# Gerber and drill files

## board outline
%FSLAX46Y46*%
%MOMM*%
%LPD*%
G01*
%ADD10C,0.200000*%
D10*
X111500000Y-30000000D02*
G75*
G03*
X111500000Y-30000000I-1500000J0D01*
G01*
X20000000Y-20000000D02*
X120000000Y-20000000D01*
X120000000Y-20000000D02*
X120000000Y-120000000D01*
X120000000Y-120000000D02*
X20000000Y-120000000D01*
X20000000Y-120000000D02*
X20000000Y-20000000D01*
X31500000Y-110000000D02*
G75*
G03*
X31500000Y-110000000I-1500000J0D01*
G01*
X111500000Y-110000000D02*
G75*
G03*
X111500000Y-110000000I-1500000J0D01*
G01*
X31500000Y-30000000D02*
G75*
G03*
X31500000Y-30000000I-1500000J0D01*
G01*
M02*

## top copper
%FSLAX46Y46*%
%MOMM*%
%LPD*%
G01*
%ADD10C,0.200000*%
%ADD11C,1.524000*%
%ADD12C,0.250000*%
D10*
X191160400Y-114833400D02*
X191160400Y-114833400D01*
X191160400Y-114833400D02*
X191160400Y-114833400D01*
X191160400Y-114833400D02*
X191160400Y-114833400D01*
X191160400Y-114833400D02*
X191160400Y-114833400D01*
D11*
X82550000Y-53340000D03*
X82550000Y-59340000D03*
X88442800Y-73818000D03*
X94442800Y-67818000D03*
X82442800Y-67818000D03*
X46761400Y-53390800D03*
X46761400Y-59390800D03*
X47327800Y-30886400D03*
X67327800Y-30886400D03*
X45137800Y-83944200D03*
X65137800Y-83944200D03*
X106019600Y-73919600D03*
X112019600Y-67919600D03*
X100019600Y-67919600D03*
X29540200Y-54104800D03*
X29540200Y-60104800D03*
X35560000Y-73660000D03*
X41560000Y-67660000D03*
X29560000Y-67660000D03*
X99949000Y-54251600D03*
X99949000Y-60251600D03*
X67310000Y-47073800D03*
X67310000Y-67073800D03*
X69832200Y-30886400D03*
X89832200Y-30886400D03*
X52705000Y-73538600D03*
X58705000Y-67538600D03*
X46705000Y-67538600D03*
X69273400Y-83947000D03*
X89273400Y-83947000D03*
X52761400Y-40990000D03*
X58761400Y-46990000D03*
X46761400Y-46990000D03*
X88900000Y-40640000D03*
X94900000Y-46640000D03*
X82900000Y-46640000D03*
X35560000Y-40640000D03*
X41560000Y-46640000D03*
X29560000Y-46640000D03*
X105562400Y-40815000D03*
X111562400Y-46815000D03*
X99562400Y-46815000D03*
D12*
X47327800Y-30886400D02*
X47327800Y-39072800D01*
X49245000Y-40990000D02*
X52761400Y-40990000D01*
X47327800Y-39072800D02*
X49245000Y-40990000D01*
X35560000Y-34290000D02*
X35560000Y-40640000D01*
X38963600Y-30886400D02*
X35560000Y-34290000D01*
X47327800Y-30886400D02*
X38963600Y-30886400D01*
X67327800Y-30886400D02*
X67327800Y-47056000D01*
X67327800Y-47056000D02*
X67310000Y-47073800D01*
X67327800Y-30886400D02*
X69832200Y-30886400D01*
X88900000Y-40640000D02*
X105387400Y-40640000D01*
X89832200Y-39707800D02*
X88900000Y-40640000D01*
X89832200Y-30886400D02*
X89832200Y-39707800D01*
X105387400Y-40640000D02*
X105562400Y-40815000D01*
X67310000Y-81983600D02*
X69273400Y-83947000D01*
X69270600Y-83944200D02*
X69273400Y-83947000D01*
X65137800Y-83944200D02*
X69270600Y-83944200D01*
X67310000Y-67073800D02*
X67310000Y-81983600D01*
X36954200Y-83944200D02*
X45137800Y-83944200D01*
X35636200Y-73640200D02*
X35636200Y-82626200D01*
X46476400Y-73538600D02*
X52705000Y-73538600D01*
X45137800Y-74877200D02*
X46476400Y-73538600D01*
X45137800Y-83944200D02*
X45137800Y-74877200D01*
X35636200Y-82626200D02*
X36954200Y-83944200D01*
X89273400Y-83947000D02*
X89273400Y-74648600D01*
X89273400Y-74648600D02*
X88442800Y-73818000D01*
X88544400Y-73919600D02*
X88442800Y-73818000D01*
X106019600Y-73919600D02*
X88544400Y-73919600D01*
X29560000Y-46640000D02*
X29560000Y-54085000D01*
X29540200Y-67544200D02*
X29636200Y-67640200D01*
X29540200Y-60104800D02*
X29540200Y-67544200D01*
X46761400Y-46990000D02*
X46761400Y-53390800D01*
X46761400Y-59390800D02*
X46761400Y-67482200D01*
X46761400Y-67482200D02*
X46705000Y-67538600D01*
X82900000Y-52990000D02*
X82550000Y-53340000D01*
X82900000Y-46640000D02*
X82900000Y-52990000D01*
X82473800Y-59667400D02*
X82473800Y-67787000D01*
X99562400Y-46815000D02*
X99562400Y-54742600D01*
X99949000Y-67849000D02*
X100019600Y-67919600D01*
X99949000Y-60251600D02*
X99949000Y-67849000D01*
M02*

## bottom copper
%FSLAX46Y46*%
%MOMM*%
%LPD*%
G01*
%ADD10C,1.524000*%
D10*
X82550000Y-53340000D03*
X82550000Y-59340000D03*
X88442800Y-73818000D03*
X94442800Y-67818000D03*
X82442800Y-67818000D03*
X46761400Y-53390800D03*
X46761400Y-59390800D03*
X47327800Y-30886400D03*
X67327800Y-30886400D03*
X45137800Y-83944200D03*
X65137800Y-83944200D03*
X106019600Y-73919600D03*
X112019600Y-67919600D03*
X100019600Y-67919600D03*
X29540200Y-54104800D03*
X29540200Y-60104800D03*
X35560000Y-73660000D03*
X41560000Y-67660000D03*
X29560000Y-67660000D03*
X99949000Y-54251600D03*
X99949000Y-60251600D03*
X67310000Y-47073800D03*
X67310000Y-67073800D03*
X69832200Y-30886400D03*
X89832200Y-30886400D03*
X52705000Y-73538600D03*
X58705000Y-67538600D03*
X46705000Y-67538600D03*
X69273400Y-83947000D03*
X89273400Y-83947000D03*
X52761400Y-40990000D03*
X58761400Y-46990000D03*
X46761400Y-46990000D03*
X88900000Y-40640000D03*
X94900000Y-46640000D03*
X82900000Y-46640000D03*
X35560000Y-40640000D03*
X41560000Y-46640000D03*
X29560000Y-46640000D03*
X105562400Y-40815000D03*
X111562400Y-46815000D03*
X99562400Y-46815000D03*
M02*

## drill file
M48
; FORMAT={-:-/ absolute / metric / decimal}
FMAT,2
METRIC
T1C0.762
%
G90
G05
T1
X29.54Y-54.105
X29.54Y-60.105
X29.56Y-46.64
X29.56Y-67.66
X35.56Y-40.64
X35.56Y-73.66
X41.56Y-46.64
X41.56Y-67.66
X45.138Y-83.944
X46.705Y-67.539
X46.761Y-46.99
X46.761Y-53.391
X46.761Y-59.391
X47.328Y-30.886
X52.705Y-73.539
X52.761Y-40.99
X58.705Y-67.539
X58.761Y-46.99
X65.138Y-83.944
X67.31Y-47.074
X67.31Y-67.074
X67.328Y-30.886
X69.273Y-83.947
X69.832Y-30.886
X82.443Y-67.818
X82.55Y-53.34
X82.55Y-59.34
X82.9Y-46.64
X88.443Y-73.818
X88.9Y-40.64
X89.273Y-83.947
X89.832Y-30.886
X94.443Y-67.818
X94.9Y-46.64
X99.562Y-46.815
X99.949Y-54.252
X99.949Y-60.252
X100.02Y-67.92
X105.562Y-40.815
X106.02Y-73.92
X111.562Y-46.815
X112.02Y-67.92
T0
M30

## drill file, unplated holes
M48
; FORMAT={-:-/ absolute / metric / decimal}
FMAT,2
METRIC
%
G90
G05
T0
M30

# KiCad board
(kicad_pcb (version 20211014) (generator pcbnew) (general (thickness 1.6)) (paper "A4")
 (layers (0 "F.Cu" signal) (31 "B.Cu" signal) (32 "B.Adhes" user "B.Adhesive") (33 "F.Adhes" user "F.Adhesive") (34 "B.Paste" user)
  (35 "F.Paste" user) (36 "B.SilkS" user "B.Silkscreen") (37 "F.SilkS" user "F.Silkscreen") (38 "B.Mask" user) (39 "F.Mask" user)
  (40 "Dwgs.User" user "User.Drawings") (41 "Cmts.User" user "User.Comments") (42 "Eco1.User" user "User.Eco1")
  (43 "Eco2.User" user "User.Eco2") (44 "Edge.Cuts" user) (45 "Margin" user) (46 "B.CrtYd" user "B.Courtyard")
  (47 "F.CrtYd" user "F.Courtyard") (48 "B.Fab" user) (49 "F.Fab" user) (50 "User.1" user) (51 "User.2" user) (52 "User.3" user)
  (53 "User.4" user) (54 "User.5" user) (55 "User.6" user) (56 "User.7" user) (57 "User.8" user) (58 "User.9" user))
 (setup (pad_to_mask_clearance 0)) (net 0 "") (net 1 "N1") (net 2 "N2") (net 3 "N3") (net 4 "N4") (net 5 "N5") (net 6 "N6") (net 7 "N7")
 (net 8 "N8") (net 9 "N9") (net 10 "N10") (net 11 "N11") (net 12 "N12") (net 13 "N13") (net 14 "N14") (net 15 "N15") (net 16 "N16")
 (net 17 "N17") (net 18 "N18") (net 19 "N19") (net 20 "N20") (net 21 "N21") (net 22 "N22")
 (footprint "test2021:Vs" (layer "F.Cu") (at 82.55 56.34)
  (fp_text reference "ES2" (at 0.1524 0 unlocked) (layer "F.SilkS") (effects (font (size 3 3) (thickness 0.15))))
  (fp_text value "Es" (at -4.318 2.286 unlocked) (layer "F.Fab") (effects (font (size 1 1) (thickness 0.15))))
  (pad "1" thru_hole circle (at 0 -3) (size 1.524 1.524) (drill 0.762) (layers *.Cu *.Mask) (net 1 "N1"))
  (pad "2" thru_hole circle (at 0 3) (size 1.524 1.524) (drill 0.762) (layers *.Cu *.Mask) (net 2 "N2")))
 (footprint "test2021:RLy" (layer "F.Cu") (at 88.4428 67.818 180)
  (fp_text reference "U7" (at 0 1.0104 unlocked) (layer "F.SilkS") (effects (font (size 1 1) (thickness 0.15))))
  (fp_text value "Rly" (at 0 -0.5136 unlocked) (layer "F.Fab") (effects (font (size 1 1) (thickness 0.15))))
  (pad "1" thru_hole circle (at 0 -6 180) (size 1.524 1.524) (drill 0.762) (layers *.Cu *.Mask) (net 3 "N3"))
  (pad "2" thru_hole circle (at -6 0 180) (size 1.524 1.524) (drill 0.762) (layers *.Cu *.Mask) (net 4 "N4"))
  (pad "3" thru_hole circle (at 6 0 180) (size 1.524 1.524) (drill 0.762) (layers *.Cu *.Mask) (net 2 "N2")))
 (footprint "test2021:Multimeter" (layer "F.Cu") (at 46.7614 56.3908)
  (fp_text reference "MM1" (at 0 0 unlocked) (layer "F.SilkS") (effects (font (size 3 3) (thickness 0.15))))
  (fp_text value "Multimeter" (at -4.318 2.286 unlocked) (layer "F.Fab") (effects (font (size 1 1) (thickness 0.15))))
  (pad "1" thru_hole circle (at 0 -3) (size 1.524 1.524) (drill 0.762) (layers *.Cu *.Mask) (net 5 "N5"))
  (pad "2" thru_hole circle (at 0 3) (size 1.524 1.524) (drill 0.762) (layers *.Cu *.Mask) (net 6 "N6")))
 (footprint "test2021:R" (layer "F.Cu") (at 57.3278 30.8864)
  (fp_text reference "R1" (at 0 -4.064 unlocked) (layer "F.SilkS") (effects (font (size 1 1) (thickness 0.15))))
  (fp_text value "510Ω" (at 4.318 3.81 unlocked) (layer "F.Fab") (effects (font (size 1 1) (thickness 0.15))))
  (pad "1" thru_hole circle (at -10 0) (size 1.524 1.524) (drill 0.762) (layers *.Cu *.Mask) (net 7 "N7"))
  (pad "2" thru_hole circle (at 10 0) (size 1.524 1.524) (drill 0.762) (layers *.Cu *.Mask) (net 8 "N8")))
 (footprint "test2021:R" (layer "F.Cu") (at 55.1378 83.9442)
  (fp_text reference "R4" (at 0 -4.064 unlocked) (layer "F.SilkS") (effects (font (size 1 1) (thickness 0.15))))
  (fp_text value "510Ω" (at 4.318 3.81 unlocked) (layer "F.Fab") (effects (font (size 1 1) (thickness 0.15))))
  (pad "1" thru_hole circle (at -10 0) (size 1.524 1.524) (drill 0.762) (layers *.Cu *.Mask) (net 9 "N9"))
  (pad "2" thru_hole circle (at 10 0) (size 1.524 1.524) (drill 0.762) (layers *.Cu *.Mask) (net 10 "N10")))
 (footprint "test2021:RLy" (layer "F.Cu") (at 106.0196 67.9196 180)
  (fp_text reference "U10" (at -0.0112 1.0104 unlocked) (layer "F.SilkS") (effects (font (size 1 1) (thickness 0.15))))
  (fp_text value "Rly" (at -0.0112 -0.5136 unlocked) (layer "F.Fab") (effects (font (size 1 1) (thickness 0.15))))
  (pad "1" thru_hole circle (at 0 -6 180) (size 1.524 1.524) (drill 0.762) (layers *.Cu *.Mask) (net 3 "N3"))
  (pad "2" thru_hole circle (at -6 0 180) (size 1.524 1.524) (drill 0.762) (layers *.Cu *.Mask) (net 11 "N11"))
  (pad "3" thru_hole circle (at 6 0 180) (size 1.524 1.524) (drill 0.762) (layers *.Cu *.Mask) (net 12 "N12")))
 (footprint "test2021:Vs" (layer "F.Cu") (at 29.5402 57.1048)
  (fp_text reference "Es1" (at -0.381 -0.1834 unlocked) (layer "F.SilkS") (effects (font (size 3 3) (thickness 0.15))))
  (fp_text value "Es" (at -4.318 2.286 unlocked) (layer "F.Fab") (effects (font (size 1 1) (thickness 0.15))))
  (pad "1" thru_hole circle (at 0 -3) (size 1.524 1.524) (drill 0.762) (layers *.Cu *.Mask) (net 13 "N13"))
  (pad "2" thru_hole circle (at 0 3) (size 1.524 1.524) (drill 0.762) (layers *.Cu *.Mask) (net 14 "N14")))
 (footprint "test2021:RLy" (layer "F.Cu") (at 35.56 67.66 180)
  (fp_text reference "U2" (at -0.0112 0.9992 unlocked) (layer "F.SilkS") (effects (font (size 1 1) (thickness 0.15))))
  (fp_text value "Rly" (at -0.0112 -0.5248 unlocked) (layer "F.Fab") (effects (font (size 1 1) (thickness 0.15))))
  (pad "1" thru_hole circle (at 0 -6 180) (size 1.524 1.524) (drill 0.762) (layers *.Cu *.Mask) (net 9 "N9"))
  (pad "2" thru_hole circle (at -6 0 180) (size 1.524 1.524) (drill 0.762) (layers *.Cu *.Mask) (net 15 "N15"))
  (pad "3" thru_hole circle (at 6 0 180) (size 1.524 1.524) (drill 0.762) (layers *.Cu *.Mask) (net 14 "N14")))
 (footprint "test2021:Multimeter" (layer "F.Cu") (at 99.949 57.2516)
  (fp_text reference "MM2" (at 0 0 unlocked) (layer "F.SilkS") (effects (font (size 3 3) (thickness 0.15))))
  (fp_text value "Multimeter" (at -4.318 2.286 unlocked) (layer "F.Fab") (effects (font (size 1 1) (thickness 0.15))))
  (pad "1" thru_hole circle (at 0 -3) (size 1.524 1.524) (drill 0.762) (layers *.Cu *.Mask) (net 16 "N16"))
  (pad "2" thru_hole circle (at 0 3) (size 1.524 1.524) (drill 0.762) (layers *.Cu *.Mask) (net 12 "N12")))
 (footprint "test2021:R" (layer "F.Cu") (at 67.31 57.0738 -90)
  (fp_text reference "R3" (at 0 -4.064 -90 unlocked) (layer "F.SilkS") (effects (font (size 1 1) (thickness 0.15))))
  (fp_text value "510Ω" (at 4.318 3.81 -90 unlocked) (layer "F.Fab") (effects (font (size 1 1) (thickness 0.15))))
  (pad "1" thru_hole circle (at -10 0 270) (size 1.524 1.524) (drill 0.762) (layers *.Cu *.Mask) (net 8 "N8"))
  (pad "2" thru_hole circle (at 10 0 270) (size 1.524 1.524) (drill 0.762) (layers *.Cu *.Mask) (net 10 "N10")))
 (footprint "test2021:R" (layer "F.Cu") (at 79.8322 30.8864)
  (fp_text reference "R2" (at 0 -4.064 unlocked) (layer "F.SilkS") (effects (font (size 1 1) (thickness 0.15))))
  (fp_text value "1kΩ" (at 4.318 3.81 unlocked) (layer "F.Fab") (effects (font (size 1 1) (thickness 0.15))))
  (pad "1" thru_hole circle (at -10 0) (size 1.524 1.524) (drill 0.762) (layers *.Cu *.Mask) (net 8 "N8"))
  (pad "2" thru_hole circle (at 10 0) (size 1.524 1.524) (drill 0.762) (layers *.Cu *.Mask) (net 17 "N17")))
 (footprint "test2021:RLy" (layer "F.Cu") (at 52.705 67.5386 180)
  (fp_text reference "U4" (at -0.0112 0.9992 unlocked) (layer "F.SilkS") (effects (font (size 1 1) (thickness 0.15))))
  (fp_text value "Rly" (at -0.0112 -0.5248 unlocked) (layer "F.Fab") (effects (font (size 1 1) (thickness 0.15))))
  (pad "1" thru_hole circle (at 0 -6 180) (size 1.524 1.524) (drill 0.762) (layers *.Cu *.Mask) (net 9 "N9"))
  (pad "2" thru_hole circle (at -6 0 180) (size 1.524 1.524) (drill 0.762) (layers *.Cu *.Mask) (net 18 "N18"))
  (pad "3" thru_hole circle (at 6 0 180) (size 1.524 1.524) (drill 0.762) (layers *.Cu *.Mask) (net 6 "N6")))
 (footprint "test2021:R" (layer "F.Cu") (at 79.2734 83.947)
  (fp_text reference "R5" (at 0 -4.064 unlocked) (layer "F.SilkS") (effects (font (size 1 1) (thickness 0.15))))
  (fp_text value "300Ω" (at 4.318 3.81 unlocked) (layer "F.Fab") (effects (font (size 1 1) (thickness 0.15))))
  (pad "1" thru_hole circle (at -10 0) (size 1.524 1.524) (drill 0.762) (layers *.Cu *.Mask) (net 10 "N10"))
  (pad "2" thru_hole circle (at 10 0) (size 1.524 1.524) (drill 0.762) (layers *.Cu *.Mask) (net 3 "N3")))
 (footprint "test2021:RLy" (layer "B.Cu") (at 52.7614 46.99 180)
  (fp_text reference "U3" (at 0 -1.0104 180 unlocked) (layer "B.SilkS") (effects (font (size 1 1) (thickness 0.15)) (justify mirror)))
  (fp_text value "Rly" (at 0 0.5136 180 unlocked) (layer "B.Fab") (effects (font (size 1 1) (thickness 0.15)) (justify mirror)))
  (pad "1" thru_hole circle (at 0 6 180) (size 1.524 1.524) (drill 0.762) (layers *.Cu *.Mask) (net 7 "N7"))
  (pad "2" thru_hole circle (at -6 0 180) (size 1.524 1.524) (drill 0.762) (layers *.Cu *.Mask) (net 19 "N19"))
  (pad "3" thru_hole circle (at 6 0 180) (size 1.524 1.524) (drill 0.762) (layers *.Cu *.Mask) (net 5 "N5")))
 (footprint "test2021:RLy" (layer "B.Cu") (at 88.9 46.64 180)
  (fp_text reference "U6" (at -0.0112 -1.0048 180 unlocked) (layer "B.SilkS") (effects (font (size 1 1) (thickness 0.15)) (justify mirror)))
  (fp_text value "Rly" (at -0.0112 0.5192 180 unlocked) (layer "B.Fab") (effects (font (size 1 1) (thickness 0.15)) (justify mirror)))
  (pad "1" thru_hole circle (at 0 6 180) (size 1.524 1.524) (drill 0.762) (layers *.Cu *.Mask) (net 17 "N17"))
  (pad "2" thru_hole circle (at -6 0 180) (size 1.524 1.524) (drill 0.762) (layers *.Cu *.Mask) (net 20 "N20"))
  (pad "3" thru_hole circle (at 6 0 180) (size 1.524 1.524) (drill 0.762) (layers *.Cu *.Mask) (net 1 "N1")))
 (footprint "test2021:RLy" (layer "B.Cu") (at 35.56 46.64 180)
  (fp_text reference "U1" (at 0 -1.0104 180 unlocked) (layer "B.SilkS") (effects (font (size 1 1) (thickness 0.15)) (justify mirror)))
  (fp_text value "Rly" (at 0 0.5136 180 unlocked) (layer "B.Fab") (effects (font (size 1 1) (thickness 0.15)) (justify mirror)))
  (pad "1" thru_hole circle (at 0 6 180) (size 1.524 1.524) (drill 0.762) (layers *.Cu *.Mask) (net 7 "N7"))
  (pad "2" thru_hole circle (at -6 0 180) (size 1.524 1.524) (drill 0.762) (layers *.Cu *.Mask) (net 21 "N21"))
  (pad "3" thru_hole circle (at 6 0 180) (size 1.524 1.524) (drill 0.762) (layers *.Cu *.Mask) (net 13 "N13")))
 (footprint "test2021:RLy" (layer "B.Cu") (at 105.5624 46.815 180)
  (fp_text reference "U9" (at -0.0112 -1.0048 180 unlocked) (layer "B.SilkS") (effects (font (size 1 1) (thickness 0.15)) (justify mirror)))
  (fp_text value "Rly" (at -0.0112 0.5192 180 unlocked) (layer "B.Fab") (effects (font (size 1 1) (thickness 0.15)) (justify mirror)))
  (pad "1" thru_hole circle (at 0 6 180) (size 1.524 1.524) (drill 0.762) (layers *.Cu *.Mask) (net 17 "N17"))
  (pad "2" thru_hole circle (at -6 0 180) (size 1.524 1.524) (drill 0.762) (layers *.Cu *.Mask) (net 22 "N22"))
  (pad "3" thru_hole circle (at 6 0 180) (size 1.524 1.524) (drill 0.762) (layers *.Cu *.Mask) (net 16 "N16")))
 (gr_rect (start 191.1604 114.8334) (end 191.1604 114.8334) (layer "F.Cu") (width 0.2) (fill none))
 (gr_circle (center 110 30) (end 111.5 30) (layer "Edge.Cuts") (width 0.2) (fill none))
 (gr_rect (start 20 20) (end 120 120) (layer "Edge.Cuts") (width 0.2) (fill none))
 (gr_circle (center 30 110) (end 31.5 110) (layer "Edge.Cuts") (width 0.2) (fill none))
 (gr_circle (center 110 110) (end 111.5 110) (layer "Edge.Cuts") (width 0.2) (fill none))
 (gr_circle (center 30 30) (end 31.5 30) (layer "Edge.Cuts") (width 0.2) (fill none))
 (segment (start 47.3278 30.8864) (end 47.3278 39.0728) (width 0.25) (layer "F.Cu") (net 7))
 (segment (start 49.245 40.99) (end 52.7614 40.99) (width 0.25) (layer "F.Cu") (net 7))
 (segment (start 47.3278 39.0728) (end 49.245 40.99) (width 0.25) (layer "F.Cu") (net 7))
 (segment (start 35.56 34.29) (end 35.56 40.64) (width 0.25) (layer "F.Cu") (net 7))
 (segment (start 38.9636 30.8864) (end 35.56 34.29) (width 0.25) (layer "F.Cu") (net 7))
 (segment (start 47.3278 30.8864) (end 38.9636 30.8864) (width 0.25) (layer "F.Cu") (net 7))
 (segment (start 67.3278 30.8864) (end 67.3278 47.056) (width 0.25) (layer "F.Cu") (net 8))
 (segment (start 67.3278 47.056) (end 67.31 47.0738) (width 0.25) (layer "F.Cu") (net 8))
 (segment (start 67.3278 30.8864) (end 69.8322 30.8864) (width 0.25) (layer "F.Cu") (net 8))
 (segment (start 88.9 40.64) (end 105.3874 40.64) (width 0.25) (layer "F.Cu") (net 17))
 (segment (start 89.8322 39.7078) (end 88.9 40.64) (width 0.25) (layer "F.Cu") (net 17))
 (segment (start 89.8322 30.8864) (end 89.8322 39.7078) (width 0.25) (layer "F.Cu") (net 17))
 (segment (start 105.3874 40.64) (end 105.5624 40.815) (width 0.25) (layer "F.Cu") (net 17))
 (segment (start 67.31 81.9836) (end 69.2734 83.947) (width 0.25) (layer "F.Cu") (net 10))
 (segment (start 69.2706 83.9442) (end 69.2734 83.947) (width 0.25) (layer "F.Cu") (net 10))
 (segment (start 65.1378 83.9442) (end 69.2706 83.9442) (width 0.25) (layer "F.Cu") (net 10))
 (segment (start 67.31 67.0738) (end 67.31 81.9836) (width 0.25) (layer "F.Cu") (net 10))
 (segment (start 36.9542 83.9442) (end 45.1378 83.9442) (width 0.25) (layer "F.Cu") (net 9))
 (segment (start 35.6362 73.6402) (end 35.6362 82.6262) (width 0.25) (layer "F.Cu") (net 9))
 (segment (start 46.4764 73.5386) (end 52.705 73.5386) (width 0.25) (layer "F.Cu") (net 9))
 (segment (start 45.1378 74.8772) (end 46.4764 73.5386) (width 0.25) (layer "F.Cu") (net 9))
 (segment (start 45.1378 83.9442) (end 45.1378 74.8772) (width 0.25) (layer "F.Cu") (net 9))
 (segment (start 35.6362 82.6262) (end 36.9542 83.9442) (width 0.25) (layer "F.Cu") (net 9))
 (segment (start 89.2734 83.947) (end 89.2734 74.6486) (width 0.25) (layer "F.Cu") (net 3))
 (segment (start 89.2734 74.6486) (end 88.4428 73.818) (width 0.25) (layer "F.Cu") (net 3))
 (segment (start 88.5444 73.9196) (end 88.4428 73.818) (width 0.25) (layer "F.Cu") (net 3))
 (segment (start 106.0196 73.9196) (end 88.5444 73.9196) (width 0.25) (layer "F.Cu") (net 3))
 (segment (start 29.56 46.64) (end 29.56 54.085) (width 0.25) (layer "F.Cu") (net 13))
 (segment (start 29.5402 67.5442) (end 29.6362 67.6402) (width 0.25) (layer "F.Cu") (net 14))
 (segment (start 29.5402 60.1048) (end 29.5402 67.5442) (width 0.25) (layer "F.Cu") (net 14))
 (segment (start 46.7614 46.99) (end 46.7614 53.3908) (width 0.25) (layer "F.Cu") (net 5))
 (segment (start 46.7614 59.3908) (end 46.7614 67.4822) (width 0.25) (layer "F.Cu") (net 6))
 (segment (start 46.7614 67.4822) (end 46.705 67.5386) (width 0.25) (layer "F.Cu") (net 6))
 (segment (start 82.9 52.99) (end 82.55 53.34) (width 0.25) (layer "F.Cu") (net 1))
 (segment (start 82.9 46.64) (end 82.9 52.99) (width 0.25) (layer "F.Cu") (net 1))
 (segment (start 82.4738 59.6674) (end 82.4738 67.787) (width 0.25) (layer "F.Cu") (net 2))
 (segment (start 99.5624 46.815) (end 99.5624 54.7426) (width 0.25) (layer "F.Cu") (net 16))
 (segment (start 99.949 67.849) (end 100.0196 67.9196) (width 0.25) (layer "F.Cu") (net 12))
 (segment (start 99.949 60.2516) (end 99.949 67.849) (width 0.25) (layer "F.Cu") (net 12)))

